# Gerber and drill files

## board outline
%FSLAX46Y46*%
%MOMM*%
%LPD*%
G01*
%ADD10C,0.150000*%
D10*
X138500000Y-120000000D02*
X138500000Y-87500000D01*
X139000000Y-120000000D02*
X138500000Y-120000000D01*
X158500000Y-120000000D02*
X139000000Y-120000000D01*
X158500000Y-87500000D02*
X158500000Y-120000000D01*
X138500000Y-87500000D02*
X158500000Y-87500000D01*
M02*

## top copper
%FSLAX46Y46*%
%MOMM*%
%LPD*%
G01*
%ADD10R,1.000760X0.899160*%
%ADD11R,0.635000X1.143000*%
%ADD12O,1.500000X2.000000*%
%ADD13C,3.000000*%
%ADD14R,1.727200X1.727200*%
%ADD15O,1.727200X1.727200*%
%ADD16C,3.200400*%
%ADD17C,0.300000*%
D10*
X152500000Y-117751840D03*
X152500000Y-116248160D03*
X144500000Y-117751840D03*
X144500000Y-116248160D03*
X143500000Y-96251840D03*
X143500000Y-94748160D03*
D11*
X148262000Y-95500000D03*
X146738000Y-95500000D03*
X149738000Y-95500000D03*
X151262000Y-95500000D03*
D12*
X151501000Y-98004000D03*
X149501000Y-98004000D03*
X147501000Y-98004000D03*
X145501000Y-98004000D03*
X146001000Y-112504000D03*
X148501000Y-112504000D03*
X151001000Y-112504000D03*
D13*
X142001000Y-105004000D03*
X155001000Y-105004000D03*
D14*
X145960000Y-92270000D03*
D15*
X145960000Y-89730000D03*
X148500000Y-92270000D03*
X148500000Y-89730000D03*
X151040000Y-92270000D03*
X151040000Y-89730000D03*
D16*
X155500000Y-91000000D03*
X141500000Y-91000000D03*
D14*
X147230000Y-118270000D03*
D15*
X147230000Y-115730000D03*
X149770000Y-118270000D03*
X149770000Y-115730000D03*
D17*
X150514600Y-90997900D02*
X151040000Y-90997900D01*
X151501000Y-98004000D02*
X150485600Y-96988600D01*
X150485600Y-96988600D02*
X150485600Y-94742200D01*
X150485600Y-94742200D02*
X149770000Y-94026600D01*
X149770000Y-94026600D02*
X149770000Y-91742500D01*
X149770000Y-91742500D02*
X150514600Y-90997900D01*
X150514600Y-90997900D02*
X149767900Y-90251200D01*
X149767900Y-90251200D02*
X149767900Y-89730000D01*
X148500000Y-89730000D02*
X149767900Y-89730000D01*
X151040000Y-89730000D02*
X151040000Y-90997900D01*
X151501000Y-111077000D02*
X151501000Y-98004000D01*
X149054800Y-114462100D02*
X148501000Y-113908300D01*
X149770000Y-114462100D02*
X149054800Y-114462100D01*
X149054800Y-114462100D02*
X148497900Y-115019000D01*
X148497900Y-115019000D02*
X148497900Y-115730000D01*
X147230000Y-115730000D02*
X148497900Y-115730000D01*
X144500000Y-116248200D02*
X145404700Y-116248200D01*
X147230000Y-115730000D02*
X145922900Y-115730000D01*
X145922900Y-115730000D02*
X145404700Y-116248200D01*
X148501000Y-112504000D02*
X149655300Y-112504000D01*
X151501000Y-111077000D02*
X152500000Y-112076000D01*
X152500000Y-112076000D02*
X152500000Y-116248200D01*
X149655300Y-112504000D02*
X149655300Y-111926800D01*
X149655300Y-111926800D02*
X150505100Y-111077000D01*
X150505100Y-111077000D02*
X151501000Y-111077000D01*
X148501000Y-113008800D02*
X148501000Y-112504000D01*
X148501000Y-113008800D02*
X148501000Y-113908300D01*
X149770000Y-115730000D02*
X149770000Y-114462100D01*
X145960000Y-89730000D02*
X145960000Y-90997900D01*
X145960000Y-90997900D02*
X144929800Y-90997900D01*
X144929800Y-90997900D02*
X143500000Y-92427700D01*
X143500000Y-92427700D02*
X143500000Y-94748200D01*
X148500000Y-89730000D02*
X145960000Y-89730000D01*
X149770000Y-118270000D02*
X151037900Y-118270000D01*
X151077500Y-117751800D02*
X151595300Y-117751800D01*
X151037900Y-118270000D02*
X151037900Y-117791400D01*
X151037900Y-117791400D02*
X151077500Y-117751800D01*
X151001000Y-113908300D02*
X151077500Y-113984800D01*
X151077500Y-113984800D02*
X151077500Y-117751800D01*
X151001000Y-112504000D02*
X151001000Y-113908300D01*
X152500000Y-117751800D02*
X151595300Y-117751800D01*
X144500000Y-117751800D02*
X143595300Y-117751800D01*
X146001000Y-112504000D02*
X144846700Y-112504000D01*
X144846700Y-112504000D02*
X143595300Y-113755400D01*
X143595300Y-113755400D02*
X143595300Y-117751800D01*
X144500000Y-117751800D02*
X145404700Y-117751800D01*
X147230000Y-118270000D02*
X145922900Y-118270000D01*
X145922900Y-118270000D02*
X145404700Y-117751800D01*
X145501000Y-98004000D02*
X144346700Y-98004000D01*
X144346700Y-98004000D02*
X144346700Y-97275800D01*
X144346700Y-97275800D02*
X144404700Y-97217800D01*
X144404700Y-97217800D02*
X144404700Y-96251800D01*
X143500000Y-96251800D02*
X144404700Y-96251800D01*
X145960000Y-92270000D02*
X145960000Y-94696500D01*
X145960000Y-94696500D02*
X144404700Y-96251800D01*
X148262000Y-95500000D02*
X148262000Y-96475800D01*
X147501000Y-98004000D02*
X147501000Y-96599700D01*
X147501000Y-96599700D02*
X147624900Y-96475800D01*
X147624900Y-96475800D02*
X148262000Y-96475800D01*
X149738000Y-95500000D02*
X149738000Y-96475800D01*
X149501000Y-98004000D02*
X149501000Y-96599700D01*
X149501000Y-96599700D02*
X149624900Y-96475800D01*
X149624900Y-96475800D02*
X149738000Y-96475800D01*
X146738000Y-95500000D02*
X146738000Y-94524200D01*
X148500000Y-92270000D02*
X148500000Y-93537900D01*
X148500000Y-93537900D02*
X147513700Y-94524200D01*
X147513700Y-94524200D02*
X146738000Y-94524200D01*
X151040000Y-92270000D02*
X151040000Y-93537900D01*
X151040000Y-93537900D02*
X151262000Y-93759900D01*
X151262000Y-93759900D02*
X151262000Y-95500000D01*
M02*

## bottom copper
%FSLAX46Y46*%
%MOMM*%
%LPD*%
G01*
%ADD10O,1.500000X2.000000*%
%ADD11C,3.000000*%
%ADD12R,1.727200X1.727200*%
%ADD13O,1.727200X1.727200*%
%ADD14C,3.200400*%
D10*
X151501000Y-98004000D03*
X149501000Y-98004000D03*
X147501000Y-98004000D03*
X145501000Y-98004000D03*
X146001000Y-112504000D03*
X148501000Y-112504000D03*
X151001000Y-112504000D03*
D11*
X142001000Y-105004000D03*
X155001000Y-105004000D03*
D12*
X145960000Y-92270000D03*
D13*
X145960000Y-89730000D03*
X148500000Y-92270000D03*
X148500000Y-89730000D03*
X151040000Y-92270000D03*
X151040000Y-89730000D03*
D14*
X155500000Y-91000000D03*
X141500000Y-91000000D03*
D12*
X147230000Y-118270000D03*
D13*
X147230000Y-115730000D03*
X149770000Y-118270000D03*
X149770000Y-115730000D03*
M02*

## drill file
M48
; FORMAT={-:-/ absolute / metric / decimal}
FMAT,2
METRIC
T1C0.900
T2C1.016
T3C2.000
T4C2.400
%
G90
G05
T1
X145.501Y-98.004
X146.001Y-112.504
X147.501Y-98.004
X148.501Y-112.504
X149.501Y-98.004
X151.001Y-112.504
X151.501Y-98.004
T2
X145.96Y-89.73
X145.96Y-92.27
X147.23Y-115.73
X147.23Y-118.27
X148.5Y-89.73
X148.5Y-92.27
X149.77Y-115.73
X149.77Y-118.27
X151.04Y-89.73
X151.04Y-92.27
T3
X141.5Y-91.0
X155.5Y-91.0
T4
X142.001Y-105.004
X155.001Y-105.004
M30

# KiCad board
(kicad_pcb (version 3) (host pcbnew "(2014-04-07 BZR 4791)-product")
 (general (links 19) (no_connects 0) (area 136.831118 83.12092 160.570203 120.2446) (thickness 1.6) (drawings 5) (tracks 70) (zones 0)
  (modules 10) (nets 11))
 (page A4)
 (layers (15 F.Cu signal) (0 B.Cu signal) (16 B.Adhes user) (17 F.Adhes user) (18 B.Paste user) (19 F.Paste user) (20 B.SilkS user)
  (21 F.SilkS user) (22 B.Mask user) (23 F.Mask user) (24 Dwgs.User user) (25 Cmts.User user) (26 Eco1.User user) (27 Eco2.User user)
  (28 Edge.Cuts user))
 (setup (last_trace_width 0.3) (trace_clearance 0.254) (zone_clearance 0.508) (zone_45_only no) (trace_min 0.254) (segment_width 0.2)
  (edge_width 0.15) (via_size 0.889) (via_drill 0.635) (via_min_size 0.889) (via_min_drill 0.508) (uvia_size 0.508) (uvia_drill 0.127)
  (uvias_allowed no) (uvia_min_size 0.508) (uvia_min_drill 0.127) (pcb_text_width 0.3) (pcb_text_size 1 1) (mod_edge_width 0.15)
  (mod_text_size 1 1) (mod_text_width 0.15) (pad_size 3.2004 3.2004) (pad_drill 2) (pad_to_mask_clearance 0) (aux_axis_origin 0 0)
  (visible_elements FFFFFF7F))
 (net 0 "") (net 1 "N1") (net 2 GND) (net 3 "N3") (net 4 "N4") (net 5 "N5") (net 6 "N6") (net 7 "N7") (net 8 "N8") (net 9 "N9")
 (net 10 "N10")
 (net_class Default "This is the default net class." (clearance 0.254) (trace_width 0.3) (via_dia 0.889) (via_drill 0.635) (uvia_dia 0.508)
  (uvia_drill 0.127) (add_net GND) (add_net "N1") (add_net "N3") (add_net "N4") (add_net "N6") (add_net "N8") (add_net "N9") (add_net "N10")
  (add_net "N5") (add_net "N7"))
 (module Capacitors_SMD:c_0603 (layer F.Cu) (at 152.5 117 270)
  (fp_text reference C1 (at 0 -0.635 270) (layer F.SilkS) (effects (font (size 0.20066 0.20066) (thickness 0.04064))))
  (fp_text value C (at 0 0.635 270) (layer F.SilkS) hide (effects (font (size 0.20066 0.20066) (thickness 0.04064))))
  (pad 1 smd rect (at 0.75184 0 270) (size 0.89916 1.00076) (layers F.Cu F.Paste F.Mask) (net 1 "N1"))
  (pad 2 smd rect (at -0.75184 0 270) (size 0.89916 1.00076) (layers F.Cu F.Paste F.Mask) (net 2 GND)))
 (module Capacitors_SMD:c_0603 (layer F.Cu) (at 144.5 117 270)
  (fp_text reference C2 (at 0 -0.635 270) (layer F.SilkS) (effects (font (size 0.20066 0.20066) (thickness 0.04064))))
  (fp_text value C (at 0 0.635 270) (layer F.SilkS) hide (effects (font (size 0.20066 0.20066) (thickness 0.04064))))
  (pad 1 smd rect (at 0.75184 0 270) (size 0.89916 1.00076) (layers F.Cu F.Paste F.Mask) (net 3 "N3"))
  (pad 2 smd rect (at -0.75184 0 270) (size 0.89916 1.00076) (layers F.Cu F.Paste F.Mask) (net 2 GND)))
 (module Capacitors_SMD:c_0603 (layer F.Cu) (at 143.5 95.5 270)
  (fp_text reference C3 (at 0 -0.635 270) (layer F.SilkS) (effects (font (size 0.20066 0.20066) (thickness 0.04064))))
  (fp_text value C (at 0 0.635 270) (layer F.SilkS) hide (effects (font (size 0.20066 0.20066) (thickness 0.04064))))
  (pad 1 smd rect (at 0.75184 0 270) (size 0.89916 1.00076) (layers F.Cu F.Paste F.Mask) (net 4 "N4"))
  (pad 2 smd rect (at -0.75184 0 270) (size 0.89916 1.00076) (layers F.Cu F.Paste F.Mask) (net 2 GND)))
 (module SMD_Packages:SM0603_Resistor (layer F.Cu) (at 147.5 95.5 180)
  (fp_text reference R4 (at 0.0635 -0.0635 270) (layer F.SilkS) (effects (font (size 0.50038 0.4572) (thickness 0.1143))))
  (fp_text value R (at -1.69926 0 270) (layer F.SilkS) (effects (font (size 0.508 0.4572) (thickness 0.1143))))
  (pad 1 smd rect (at -0.762 0 180) (size 0.635 1.143) (layers F.Cu F.Paste F.Mask) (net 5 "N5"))
  (pad 2 smd rect (at 0.762 0 180) (size 0.635 1.143) (layers F.Cu F.Paste F.Mask) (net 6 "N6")))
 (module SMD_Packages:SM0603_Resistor (layer F.Cu) (at 150.5 95.5)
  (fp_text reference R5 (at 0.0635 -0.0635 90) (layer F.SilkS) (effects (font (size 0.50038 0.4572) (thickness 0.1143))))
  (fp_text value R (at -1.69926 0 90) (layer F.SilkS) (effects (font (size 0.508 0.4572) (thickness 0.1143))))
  (pad 1 smd rect (at -0.762 0) (size 0.635 1.143) (layers F.Cu F.Paste F.Mask) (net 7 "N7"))
  (pad 2 smd rect (at 0.762 0) (size 0.635 1.143) (layers F.Cu F.Paste F.Mask) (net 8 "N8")))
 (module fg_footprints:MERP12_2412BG (layer F.Cu) (at 148.501 105.004)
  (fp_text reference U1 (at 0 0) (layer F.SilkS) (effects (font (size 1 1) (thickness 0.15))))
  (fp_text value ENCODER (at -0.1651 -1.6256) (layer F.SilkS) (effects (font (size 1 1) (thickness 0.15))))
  (pad 1 thru_hole oval (at 3 -7) (size 1.5 2) (drill 0.9) (layers *.Cu *.Mask F.SilkS) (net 2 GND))
  (pad 2 thru_hole oval (at 1 -7) (size 1.5 2) (drill 0.9) (layers *.Cu *.Mask F.SilkS) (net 7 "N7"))
  (pad 3 thru_hole oval (at -1 -7) (size 1.5 2) (drill 0.9) (layers *.Cu *.Mask F.SilkS) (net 5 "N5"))
  (pad 4 thru_hole oval (at -3 -7) (size 1.5 2) (drill 0.9) (layers *.Cu *.Mask F.SilkS) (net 4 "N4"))
  (pad 5 thru_hole oval (at -2.5 7.5) (size 1.5 2) (drill 0.9) (layers *.Cu *.Mask F.SilkS) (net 3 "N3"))
  (pad 6 thru_hole oval (at 0 7.5) (size 1.5 2) (drill 0.9) (layers *.Cu *.Mask F.SilkS) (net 2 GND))
  (pad 7 thru_hole oval (at 2.5 7.5) (size 1.5 2) (drill 0.9) (layers *.Cu *.Mask F.SilkS) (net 1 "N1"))
  (pad "" thru_hole circle (at -6.5 0) (size 3 3) (drill 2.4) (layers *.Cu *.Mask F.SilkS))
  (pad "" thru_hole circle (at 6.5 0) (size 3 3) (drill 2.4) (layers *.Cu *.Mask F.SilkS)))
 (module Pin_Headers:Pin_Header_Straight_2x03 (layer F.Cu) (at 148.5 91)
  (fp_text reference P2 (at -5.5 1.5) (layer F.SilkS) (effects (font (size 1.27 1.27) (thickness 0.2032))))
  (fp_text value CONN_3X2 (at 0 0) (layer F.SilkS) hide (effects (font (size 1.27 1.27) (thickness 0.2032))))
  (pad 1 thru_hole rect (at -2.54 1.27) (size 1.7272 1.7272) (drill 1.016) (layers *.Cu *.Mask F.SilkS) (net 4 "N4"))
  (pad 2 thru_hole oval (at -2.54 -1.27) (size 1.7272 1.7272) (drill 1.016) (layers *.Cu *.Mask F.SilkS) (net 2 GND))
  (pad 3 thru_hole oval (at 0 1.27) (size 1.7272 1.7272) (drill 1.016) (layers *.Cu *.Mask F.SilkS) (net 6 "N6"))
  (pad 4 thru_hole oval (at 0 -1.27) (size 1.7272 1.7272) (drill 1.016) (layers *.Cu *.Mask F.SilkS) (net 2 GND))
  (pad 5 thru_hole oval (at 2.54 1.27) (size 1.7272 1.7272) (drill 1.016) (layers *.Cu *.Mask F.SilkS) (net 8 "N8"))
  (pad 6 thru_hole oval (at 2.54 -1.27) (size 1.7272 1.7272) (drill 1.016) (layers *.Cu *.Mask F.SilkS) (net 2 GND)))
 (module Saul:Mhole (layer F.Cu) (at 155.5 91)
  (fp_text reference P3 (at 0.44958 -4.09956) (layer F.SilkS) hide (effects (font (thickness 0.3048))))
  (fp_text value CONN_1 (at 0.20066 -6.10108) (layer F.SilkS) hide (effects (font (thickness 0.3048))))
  (pad 1 thru_hole circle (at 0 0) (size 3.2004 3.2004) (drill 2) (layers *.Cu *.Mask F.SilkS) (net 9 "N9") (clearance 1.00076)))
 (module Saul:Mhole (layer F.Cu) (at 141.5 91)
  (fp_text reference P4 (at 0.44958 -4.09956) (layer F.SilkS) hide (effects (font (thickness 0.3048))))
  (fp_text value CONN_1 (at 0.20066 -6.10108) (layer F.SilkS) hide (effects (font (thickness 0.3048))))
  (pad 1 thru_hole circle (at 0 0) (size 3.2004 3.2004) (drill 2) (layers *.Cu *.Mask F.SilkS) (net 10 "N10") (clearance 1.00076)))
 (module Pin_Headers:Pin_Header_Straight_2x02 (layer F.Cu) (at 148.5 117)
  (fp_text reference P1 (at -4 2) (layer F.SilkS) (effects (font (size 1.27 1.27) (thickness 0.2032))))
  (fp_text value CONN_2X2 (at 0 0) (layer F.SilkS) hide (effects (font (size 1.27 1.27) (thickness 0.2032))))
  (pad 1 thru_hole rect (at -1.27 1.27) (size 1.7272 1.7272) (drill 1.016) (layers *.Cu *.Mask F.SilkS) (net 3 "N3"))
  (pad 2 thru_hole oval (at -1.27 -1.27) (size 1.7272 1.7272) (drill 1.016) (layers *.Cu *.Mask F.SilkS) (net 2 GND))
  (pad 3 thru_hole oval (at 1.27 1.27) (size 1.7272 1.7272) (drill 1.016) (layers *.Cu *.Mask F.SilkS) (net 1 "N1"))
  (pad 4 thru_hole oval (at 1.27 -1.27) (size 1.7272 1.7272) (drill 1.016) (layers *.Cu *.Mask F.SilkS) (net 2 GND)))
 (gr_line (start 138.5 120) (end 138.5 87.5) (angle 90) (layer Edge.Cuts) (width 0.15))
 (gr_line (start 139 120) (end 138.5 120) (angle 90) (layer Edge.Cuts) (width 0.15))
 (gr_line (start 158.5 120) (end 139 120) (angle 90) (layer Edge.Cuts) (width 0.15))
 (gr_line (start 158.5 87.5) (end 158.5 120) (angle 90) (layer Edge.Cuts) (width 0.15))
 (gr_line (start 138.5 87.5) (end 158.5 87.5) (angle 90) (layer Edge.Cuts) (width 0.15))
 (segment (start 150.5146 90.9979) (end 151.04 90.9979) (width 0.3) (layer F.Cu) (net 2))
 (segment (start 151.501 98.004) (end 150.4856 96.9886) (width 0.3) (layer F.Cu) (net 2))
 (segment (start 150.4856 96.9886) (end 150.4856 94.7422) (width 0.3) (layer F.Cu) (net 2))
 (segment (start 150.4856 94.7422) (end 149.77 94.0266) (width 0.3) (layer F.Cu) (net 2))
 (segment (start 149.77 94.0266) (end 149.77 91.7425) (width 0.3) (layer F.Cu) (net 2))
 (segment (start 149.77 91.7425) (end 150.5146 90.9979) (width 0.3) (layer F.Cu) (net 2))
 (segment (start 150.5146 90.9979) (end 149.7679 90.2512) (width 0.3) (layer F.Cu) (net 2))
 (segment (start 149.7679 90.2512) (end 149.7679 89.73) (width 0.3) (layer F.Cu) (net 2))
 (segment (start 148.5 89.73) (end 149.7679 89.73) (width 0.3) (layer F.Cu) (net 2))
 (segment (start 151.04 89.73) (end 151.04 90.9979) (width 0.3) (layer F.Cu) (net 2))
 (segment (start 151.501 111.077) (end 151.501 98.004) (width 0.3) (layer F.Cu) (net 2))
 (segment (start 149.0548 114.4621) (end 148.501 113.9083) (width 0.3) (layer F.Cu) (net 2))
 (segment (start 149.77 114.4621) (end 149.0548 114.4621) (width 0.3) (layer F.Cu) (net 2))
 (segment (start 149.0548 114.4621) (end 148.4979 115.019) (width 0.3) (layer F.Cu) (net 2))
 (segment (start 148.4979 115.019) (end 148.4979 115.73) (width 0.3) (layer F.Cu) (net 2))
 (segment (start 147.23 115.73) (end 148.4979 115.73) (width 0.3) (layer F.Cu) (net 2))
 (segment (start 144.5 116.2482) (end 145.4047 116.2482) (width 0.3) (layer F.Cu) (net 2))
 (segment (start 147.23 115.73) (end 145.9229 115.73) (width 0.3) (layer F.Cu) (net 2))
 (segment (start 145.9229 115.73) (end 145.4047 116.2482) (width 0.3) (layer F.Cu) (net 2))
 (segment (start 148.501 112.504) (end 149.6553 112.504) (width 0.3) (layer F.Cu) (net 2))
 (segment (start 151.501 111.077) (end 152.5 112.076) (width 0.3) (layer F.Cu) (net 2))
 (segment (start 152.5 112.076) (end 152.5 116.2482) (width 0.3) (layer F.Cu) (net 2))
 (segment (start 149.6553 112.504) (end 149.6553 111.9268) (width 0.3) (layer F.Cu) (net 2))
 (segment (start 149.6553 111.9268) (end 150.5051 111.077) (width 0.3) (layer F.Cu) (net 2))
 (segment (start 150.5051 111.077) (end 151.501 111.077) (width 0.3) (layer F.Cu) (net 2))
 (segment (start 148.501 113.0088) (end 148.501 112.504) (width 0.3) (layer F.Cu) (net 2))
 (segment (start 148.501 113.0088) (end 148.501 113.9083) (width 0.3) (layer F.Cu) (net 2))
 (segment (start 149.77 115.73) (end 149.77 114.4621) (width 0.3) (layer F.Cu) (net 2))
 (segment (start 145.96 89.73) (end 145.96 90.9979) (width 0.3) (layer F.Cu) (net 2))
 (segment (start 145.96 90.9979) (end 144.9298 90.9979) (width 0.3) (layer F.Cu) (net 2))
 (segment (start 144.9298 90.9979) (end 143.5 92.4277) (width 0.3) (layer F.Cu) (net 2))
 (segment (start 143.5 92.4277) (end 143.5 94.7482) (width 0.3) (layer F.Cu) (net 2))
 (segment (start 148.5 89.73) (end 145.96 89.73) (width 0.3) (layer F.Cu) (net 2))
 (segment (start 149.77 118.27) (end 151.0379 118.27) (width 0.3) (layer F.Cu) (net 1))
 (segment (start 151.0775 117.7518) (end 151.5953 117.7518) (width 0.3) (layer F.Cu) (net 1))
 (segment (start 151.0379 118.27) (end 151.0379 117.7914) (width 0.3) (layer F.Cu) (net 1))
 (segment (start 151.0379 117.7914) (end 151.0775 117.7518) (width 0.3) (layer F.Cu) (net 1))
 (segment (start 151.001 113.9083) (end 151.0775 113.9848) (width 0.3) (layer F.Cu) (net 1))
 (segment (start 151.0775 113.9848) (end 151.0775 117.7518) (width 0.3) (layer F.Cu) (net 1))
 (segment (start 151.001 112.504) (end 151.001 113.9083) (width 0.3) (layer F.Cu) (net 1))
 (segment (start 152.5 117.7518) (end 151.5953 117.7518) (width 0.3) (layer F.Cu) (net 1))
 (segment (start 144.5 117.7518) (end 143.5953 117.7518) (width 0.3) (layer F.Cu) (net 3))
 (segment (start 146.001 112.504) (end 144.8467 112.504) (width 0.3) (layer F.Cu) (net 3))
 (segment (start 144.8467 112.504) (end 143.5953 113.7554) (width 0.3) (layer F.Cu) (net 3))
 (segment (start 143.5953 113.7554) (end 143.5953 117.7518) (width 0.3) (layer F.Cu) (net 3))
 (segment (start 144.5 117.7518) (end 145.4047 117.7518) (width 0.3) (layer F.Cu) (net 3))
 (segment (start 147.23 118.27) (end 145.9229 118.27) (width 0.3) (layer F.Cu) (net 3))
 (segment (start 145.9229 118.27) (end 145.4047 117.7518) (width 0.3) (layer F.Cu) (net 3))
 (segment (start 145.501 98.004) (end 144.3467 98.004) (width 0.3) (layer F.Cu) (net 4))
 (segment (start 144.3467 98.004) (end 144.3467 97.2758) (width 0.3) (layer F.Cu) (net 4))
 (segment (start 144.3467 97.2758) (end 144.4047 97.2178) (width 0.3) (layer F.Cu) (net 4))
 (segment (start 144.4047 97.2178) (end 144.4047 96.2518) (width 0.3) (layer F.Cu) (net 4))
 (segment (start 143.5 96.2518) (end 144.4047 96.2518) (width 0.3) (layer F.Cu) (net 4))
 (segment (start 145.96 92.27) (end 145.96 94.6965) (width 0.3) (layer F.Cu) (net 4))
 (segment (start 145.96 94.6965) (end 144.4047 96.2518) (width 0.3) (layer F.Cu) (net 4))
 (segment (start 148.262 95.5) (end 148.262 96.4758) (width 0.3) (layer F.Cu) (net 5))
 (segment (start 147.501 98.004) (end 147.501 96.5997) (width 0.3) (layer F.Cu) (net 5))
 (segment (start 147.501 96.5997) (end 147.6249 96.4758) (width 0.3) (layer F.Cu) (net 5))
 (segment (start 147.6249 96.4758) (end 148.262 96.4758) (width 0.3) (layer F.Cu) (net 5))
 (segment (start 149.738 95.5) (end 149.738 96.4758) (width 0.3) (layer F.Cu) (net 7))
 (segment (start 149.501 98.004) (end 149.501 96.5997) (width 0.3) (layer F.Cu) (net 7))
 (segment (start 149.501 96.5997) (end 149.6249 96.4758) (width 0.3) (layer F.Cu) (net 7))
 (segment (start 149.6249 96.4758) (end 149.738 96.4758) (width 0.3) (layer F.Cu) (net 7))
 (segment (start 146.738 95.5) (end 146.738 94.5242) (width 0.3) (layer F.Cu) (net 6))
 (segment (start 148.5 92.27) (end 148.5 93.5379) (width 0.3) (layer F.Cu) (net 6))
 (segment (start 148.5 93.5379) (end 147.5137 94.5242) (width 0.3) (layer F.Cu) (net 6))
 (segment (start 147.5137 94.5242) (end 146.738 94.5242) (width 0.3) (layer F.Cu) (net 6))
 (segment (start 151.04 92.27) (end 151.04 93.5379) (width 0.3) (layer F.Cu) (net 8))
 (segment (start 151.04 93.5379) (end 151.262 93.7599) (width 0.3) (layer F.Cu) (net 8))
 (segment (start 151.262 93.7599) (end 151.262 95.5) (width 0.3) (layer F.Cu) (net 8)))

